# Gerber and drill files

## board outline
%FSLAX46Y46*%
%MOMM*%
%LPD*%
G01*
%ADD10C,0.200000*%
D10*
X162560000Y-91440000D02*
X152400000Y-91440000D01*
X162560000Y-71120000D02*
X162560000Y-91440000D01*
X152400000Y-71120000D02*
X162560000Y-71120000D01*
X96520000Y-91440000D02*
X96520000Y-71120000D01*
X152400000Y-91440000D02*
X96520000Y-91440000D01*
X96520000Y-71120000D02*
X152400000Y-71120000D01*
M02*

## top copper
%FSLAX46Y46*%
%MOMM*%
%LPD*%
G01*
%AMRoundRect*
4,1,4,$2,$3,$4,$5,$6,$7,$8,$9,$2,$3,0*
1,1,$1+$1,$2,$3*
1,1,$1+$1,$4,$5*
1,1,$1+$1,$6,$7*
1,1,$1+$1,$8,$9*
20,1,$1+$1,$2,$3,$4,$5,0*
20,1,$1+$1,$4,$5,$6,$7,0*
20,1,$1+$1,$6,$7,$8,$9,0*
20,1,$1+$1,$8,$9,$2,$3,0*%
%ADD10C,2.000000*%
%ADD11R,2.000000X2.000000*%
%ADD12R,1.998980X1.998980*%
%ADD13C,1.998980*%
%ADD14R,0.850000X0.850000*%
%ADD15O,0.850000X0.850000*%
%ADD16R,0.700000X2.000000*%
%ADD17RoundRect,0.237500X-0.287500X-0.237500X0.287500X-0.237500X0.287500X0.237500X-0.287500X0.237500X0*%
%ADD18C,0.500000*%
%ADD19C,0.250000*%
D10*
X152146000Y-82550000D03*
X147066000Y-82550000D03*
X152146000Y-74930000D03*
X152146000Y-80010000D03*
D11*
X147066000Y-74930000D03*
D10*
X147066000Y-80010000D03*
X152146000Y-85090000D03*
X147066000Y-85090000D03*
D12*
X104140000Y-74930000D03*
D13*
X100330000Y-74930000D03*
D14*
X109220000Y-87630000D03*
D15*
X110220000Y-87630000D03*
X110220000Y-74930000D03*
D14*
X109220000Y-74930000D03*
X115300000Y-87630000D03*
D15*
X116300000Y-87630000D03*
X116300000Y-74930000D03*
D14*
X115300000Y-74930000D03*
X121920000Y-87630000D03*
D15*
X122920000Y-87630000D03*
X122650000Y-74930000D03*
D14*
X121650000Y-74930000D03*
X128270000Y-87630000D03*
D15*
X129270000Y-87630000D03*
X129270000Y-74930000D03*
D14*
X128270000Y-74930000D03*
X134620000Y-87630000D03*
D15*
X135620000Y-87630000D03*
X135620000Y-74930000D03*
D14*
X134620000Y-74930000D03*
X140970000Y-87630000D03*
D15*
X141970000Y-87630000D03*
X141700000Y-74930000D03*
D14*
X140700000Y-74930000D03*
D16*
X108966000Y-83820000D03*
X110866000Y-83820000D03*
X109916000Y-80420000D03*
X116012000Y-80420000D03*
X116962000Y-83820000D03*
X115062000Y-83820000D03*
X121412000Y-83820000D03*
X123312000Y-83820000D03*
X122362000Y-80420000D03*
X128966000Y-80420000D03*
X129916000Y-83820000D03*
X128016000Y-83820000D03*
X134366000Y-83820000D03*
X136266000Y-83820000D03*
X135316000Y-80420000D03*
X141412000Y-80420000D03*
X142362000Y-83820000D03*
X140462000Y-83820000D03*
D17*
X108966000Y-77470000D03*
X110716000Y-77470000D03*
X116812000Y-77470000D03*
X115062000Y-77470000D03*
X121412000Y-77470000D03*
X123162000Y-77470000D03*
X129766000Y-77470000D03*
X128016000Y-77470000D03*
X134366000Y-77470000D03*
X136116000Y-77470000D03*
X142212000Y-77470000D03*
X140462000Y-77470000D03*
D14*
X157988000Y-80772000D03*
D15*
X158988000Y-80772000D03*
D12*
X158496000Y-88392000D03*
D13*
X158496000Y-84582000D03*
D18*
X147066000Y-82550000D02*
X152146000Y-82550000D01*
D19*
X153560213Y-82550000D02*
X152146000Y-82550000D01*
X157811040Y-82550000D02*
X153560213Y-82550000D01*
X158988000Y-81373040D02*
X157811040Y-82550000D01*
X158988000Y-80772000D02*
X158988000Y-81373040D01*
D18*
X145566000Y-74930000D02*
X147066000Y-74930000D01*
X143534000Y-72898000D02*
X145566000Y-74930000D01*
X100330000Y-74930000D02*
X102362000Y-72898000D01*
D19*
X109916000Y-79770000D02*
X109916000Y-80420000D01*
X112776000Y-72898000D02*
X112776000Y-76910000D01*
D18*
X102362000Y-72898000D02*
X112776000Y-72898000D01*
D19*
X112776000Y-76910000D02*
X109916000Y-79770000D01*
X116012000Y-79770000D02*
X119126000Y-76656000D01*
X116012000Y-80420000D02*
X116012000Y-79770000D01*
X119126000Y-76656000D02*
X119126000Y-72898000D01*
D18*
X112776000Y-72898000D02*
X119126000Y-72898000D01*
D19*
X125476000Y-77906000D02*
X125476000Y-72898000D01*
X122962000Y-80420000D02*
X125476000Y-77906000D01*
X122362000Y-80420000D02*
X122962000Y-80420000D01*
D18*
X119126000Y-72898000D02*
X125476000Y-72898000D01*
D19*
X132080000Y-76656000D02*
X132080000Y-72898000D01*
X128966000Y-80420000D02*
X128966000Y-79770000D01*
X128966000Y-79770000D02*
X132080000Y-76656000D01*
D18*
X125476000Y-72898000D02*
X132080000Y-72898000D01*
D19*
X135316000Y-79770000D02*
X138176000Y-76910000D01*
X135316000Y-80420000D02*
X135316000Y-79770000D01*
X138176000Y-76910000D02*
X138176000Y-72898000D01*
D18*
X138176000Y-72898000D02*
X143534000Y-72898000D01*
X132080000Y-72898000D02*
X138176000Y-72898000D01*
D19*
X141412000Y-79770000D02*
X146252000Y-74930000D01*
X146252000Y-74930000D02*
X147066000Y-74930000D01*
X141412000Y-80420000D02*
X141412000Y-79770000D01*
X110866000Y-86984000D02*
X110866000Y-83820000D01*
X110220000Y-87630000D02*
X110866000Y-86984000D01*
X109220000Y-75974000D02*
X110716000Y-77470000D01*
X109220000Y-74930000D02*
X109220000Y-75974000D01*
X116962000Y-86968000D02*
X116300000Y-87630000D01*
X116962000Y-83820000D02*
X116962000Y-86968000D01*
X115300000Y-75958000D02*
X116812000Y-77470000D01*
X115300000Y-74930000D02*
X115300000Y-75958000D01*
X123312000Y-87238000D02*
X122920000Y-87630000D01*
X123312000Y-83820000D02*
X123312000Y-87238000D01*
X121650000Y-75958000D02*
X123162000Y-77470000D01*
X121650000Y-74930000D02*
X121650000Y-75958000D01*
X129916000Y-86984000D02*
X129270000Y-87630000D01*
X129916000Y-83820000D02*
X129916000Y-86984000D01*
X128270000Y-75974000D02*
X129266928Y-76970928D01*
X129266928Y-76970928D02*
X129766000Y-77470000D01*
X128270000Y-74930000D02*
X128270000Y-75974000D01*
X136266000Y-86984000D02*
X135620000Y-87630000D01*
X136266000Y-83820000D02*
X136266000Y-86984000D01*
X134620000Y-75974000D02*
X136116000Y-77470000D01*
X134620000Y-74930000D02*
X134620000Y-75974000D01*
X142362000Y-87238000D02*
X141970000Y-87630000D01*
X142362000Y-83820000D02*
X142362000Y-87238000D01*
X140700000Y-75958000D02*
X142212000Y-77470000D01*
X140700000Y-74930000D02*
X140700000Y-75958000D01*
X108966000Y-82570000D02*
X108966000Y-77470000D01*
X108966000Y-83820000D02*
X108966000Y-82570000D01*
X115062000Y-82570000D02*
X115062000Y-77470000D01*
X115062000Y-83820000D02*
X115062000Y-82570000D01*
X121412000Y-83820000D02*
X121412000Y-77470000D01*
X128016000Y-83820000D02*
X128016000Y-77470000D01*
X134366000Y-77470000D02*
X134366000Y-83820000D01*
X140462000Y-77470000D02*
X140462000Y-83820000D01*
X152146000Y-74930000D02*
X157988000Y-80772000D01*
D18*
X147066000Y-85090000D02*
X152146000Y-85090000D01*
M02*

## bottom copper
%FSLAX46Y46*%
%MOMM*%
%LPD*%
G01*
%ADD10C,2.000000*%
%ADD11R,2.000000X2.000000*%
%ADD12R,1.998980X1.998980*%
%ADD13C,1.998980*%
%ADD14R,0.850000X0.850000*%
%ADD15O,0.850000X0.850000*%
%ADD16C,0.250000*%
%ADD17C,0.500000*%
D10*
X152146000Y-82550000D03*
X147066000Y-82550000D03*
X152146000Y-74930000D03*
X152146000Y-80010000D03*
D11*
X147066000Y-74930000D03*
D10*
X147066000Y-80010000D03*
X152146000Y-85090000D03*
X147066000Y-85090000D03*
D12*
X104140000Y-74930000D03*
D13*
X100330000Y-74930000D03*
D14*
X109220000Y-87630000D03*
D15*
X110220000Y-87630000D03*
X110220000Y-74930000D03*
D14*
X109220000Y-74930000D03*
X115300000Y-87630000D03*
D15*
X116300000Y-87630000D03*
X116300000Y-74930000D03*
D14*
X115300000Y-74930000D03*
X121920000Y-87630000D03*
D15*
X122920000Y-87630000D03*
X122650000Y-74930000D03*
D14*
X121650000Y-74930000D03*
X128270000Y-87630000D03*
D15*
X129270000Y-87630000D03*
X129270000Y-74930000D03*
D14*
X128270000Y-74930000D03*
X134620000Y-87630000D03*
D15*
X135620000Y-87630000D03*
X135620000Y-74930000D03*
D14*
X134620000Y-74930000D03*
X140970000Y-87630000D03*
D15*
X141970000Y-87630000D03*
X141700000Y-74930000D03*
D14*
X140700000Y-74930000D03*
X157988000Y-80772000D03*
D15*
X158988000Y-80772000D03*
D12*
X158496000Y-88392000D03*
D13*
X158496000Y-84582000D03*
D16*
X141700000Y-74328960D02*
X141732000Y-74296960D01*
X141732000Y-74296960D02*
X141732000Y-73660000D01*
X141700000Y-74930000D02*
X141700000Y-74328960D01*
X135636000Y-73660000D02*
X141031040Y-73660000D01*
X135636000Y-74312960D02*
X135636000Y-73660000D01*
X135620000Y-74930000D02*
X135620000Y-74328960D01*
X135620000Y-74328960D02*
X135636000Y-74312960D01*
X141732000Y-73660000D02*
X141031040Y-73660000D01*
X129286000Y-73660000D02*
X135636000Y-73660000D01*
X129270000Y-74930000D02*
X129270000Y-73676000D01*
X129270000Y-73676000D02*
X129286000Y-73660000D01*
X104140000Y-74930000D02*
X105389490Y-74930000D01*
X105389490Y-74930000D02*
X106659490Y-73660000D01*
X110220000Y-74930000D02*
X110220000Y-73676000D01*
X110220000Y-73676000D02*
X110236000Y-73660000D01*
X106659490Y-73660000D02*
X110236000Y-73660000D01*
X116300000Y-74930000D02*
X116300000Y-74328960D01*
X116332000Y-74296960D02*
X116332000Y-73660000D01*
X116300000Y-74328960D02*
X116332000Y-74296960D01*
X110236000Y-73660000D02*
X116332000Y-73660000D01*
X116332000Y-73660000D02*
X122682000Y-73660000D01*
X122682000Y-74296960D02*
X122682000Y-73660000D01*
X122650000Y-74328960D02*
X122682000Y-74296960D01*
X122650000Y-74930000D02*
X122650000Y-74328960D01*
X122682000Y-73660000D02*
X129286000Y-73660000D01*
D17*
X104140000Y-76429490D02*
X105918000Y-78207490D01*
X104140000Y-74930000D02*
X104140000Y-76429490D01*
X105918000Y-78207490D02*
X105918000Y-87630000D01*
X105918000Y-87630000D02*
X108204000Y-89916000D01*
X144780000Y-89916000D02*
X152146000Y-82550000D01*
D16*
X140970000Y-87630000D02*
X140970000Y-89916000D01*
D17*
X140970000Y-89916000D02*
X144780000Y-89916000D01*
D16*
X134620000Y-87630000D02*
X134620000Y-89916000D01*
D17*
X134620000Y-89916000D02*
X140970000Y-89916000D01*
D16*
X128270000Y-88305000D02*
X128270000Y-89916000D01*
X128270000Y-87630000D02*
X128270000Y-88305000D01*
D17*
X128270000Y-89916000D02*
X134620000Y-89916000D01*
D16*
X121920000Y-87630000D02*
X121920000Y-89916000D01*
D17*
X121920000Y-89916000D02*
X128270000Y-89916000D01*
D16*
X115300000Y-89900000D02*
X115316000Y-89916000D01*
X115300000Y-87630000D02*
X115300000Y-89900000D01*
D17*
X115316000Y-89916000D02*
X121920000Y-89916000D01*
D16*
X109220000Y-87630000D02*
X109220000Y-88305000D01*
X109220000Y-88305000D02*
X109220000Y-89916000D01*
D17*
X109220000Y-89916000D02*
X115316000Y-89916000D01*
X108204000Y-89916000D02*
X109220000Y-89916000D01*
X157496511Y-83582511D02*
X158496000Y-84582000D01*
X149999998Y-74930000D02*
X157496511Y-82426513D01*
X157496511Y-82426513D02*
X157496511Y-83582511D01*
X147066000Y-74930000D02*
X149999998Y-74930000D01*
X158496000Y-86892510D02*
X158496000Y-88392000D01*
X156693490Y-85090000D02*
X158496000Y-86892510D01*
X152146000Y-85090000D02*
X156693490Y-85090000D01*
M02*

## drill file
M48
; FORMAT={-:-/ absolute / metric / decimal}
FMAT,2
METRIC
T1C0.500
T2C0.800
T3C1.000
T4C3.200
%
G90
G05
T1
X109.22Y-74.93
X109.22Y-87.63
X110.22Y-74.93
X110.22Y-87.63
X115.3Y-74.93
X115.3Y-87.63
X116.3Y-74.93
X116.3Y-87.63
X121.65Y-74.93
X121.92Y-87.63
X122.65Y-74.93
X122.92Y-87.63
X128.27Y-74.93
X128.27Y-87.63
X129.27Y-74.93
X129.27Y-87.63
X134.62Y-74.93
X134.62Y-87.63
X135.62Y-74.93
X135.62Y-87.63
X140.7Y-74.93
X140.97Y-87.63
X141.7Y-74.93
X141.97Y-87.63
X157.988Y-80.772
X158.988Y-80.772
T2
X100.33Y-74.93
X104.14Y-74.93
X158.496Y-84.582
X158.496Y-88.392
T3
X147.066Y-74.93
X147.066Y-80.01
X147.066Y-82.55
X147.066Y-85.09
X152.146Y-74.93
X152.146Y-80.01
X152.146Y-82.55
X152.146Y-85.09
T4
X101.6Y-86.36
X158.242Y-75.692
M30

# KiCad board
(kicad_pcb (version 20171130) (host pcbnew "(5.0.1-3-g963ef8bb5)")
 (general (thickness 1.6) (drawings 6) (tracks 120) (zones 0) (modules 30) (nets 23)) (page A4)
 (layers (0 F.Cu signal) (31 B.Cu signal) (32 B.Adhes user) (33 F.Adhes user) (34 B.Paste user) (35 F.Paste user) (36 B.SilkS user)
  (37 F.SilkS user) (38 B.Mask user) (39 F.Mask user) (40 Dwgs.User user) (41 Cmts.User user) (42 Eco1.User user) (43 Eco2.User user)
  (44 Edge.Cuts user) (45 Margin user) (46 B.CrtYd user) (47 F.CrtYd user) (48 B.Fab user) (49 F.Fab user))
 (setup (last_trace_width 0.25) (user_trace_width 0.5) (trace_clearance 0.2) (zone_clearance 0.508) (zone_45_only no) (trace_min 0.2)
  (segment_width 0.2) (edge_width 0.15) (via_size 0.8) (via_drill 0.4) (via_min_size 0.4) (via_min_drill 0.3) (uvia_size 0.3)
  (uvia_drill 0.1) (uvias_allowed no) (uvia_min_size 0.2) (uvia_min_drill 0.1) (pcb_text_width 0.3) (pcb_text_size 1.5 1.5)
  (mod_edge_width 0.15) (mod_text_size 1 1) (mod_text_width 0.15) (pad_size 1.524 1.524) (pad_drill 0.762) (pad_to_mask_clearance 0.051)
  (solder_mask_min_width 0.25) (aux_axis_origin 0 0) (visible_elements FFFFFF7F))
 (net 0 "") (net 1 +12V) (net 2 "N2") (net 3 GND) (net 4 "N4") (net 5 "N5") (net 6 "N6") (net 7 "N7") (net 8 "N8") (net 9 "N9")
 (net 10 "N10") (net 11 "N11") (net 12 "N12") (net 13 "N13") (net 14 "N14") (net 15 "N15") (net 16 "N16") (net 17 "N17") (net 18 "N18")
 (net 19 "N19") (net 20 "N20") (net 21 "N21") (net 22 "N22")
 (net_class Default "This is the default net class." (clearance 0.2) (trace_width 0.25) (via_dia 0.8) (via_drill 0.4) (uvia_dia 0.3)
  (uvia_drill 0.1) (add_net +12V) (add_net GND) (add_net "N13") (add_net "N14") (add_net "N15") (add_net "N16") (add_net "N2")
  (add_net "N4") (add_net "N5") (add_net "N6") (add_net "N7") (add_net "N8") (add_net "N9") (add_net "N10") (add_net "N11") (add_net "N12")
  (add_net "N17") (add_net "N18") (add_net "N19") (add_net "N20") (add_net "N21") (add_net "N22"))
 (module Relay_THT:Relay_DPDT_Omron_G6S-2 (layer F.Cu) (at 147.066 74.93)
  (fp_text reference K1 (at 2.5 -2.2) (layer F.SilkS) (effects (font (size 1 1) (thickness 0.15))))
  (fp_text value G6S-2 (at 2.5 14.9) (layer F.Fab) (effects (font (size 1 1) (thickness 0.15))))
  (pad 7 thru_hole circle (at 5.08 7.62 270) (size 2 2) (drill 1) (layers *.Cu *.Mask) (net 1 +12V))
  (pad 4 thru_hole circle (at 0 7.62 270) (size 2 2) (drill 1) (layers *.Cu *.Mask) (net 1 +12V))
  (pad 10 thru_hole circle (at 5.08 0) (size 2 2) (drill 1) (layers *.Cu *.Mask) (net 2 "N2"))
  (pad 8 thru_hole circle (at 5.08 5.08) (size 2 2) (drill 1) (layers *.Cu *.Mask))
  (pad 1 thru_hole rect (at 0 0) (size 2 2) (drill 1) (layers *.Cu *.Mask) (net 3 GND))
  (pad 3 thru_hole circle (at 0 5.08) (size 2 2) (drill 1) (layers *.Cu *.Mask))
  (pad 6 thru_hole circle (at 5.08 10.16) (size 2 2) (drill 1) (layers *.Cu *.Mask) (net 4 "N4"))
  (pad 5 thru_hole circle (at 0 10.16) (size 2 2) (drill 1) (layers *.Cu *.Mask) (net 4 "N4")))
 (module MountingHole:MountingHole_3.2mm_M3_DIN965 (layer F.Cu) (at 101.6 86.36)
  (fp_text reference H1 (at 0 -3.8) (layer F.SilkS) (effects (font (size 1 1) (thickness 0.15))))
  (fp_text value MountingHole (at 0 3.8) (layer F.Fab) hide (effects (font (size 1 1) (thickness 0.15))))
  (pad 1 np_thru_hole circle (at 0 0) (size 3.2 3.2) (drill 3.2) (layers *.Cu *.Mask)))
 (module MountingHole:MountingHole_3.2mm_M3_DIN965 (layer F.Cu) (at 158.242 75.692)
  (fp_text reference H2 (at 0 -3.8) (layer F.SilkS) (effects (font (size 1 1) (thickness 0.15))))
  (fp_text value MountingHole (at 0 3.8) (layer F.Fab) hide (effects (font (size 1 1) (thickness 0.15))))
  (pad 1 np_thru_hole circle (at 0 0) (size 3.2 3.2) (drill 3.2) (layers *.Cu *.Mask)))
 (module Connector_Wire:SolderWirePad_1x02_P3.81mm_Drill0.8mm (layer F.Cu) (at 104.14 74.93 180)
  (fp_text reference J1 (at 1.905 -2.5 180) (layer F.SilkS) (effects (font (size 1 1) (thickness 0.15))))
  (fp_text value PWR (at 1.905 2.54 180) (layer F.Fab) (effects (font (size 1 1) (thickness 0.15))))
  (pad 1 thru_hole rect (at 0 0 180) (size 1.99898 1.99898) (drill 0.8001) (layers *.Cu *.Mask) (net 1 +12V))
  (pad 2 thru_hole circle (at 3.81 0 180) (size 1.99898 1.99898) (drill 0.8001) (layers *.Cu *.Mask) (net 3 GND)))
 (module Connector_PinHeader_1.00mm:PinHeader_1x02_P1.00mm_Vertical (layer F.Cu) (at 109.22 87.63 90)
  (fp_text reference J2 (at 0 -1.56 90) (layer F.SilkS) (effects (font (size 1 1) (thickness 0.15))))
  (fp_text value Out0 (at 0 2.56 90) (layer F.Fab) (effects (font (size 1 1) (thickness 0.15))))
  (pad 1 thru_hole rect (at 0 0 90) (size 0.85 0.85) (drill 0.5) (layers *.Cu *.Mask) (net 1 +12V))
  (pad 2 thru_hole oval (at 0 1 90) (size 0.85 0.85) (drill 0.5) (layers *.Cu *.Mask) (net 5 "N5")))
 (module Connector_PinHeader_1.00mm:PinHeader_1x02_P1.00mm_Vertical (layer F.Cu) (at 109.22 74.93 90)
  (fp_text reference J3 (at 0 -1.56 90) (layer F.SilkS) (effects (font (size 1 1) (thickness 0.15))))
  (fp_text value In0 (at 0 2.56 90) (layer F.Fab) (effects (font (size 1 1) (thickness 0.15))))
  (pad 2 thru_hole oval (at 0 1 90) (size 0.85 0.85) (drill 0.5) (layers *.Cu *.Mask) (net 1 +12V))
  (pad 1 thru_hole rect (at 0 0 90) (size 0.85 0.85) (drill 0.5) (layers *.Cu *.Mask) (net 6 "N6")))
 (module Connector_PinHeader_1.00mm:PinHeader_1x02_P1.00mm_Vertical (layer F.Cu) (at 115.3 87.63 90)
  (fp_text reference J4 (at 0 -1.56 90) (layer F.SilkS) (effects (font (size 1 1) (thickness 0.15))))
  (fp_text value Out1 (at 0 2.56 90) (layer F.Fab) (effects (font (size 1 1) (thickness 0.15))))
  (pad 1 thru_hole rect (at 0 0 90) (size 0.85 0.85) (drill 0.5) (layers *.Cu *.Mask) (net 1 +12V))
  (pad 2 thru_hole oval (at 0 1 90) (size 0.85 0.85) (drill 0.5) (layers *.Cu *.Mask) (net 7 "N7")))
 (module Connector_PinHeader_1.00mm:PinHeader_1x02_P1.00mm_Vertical (layer F.Cu) (at 115.3 74.93 90)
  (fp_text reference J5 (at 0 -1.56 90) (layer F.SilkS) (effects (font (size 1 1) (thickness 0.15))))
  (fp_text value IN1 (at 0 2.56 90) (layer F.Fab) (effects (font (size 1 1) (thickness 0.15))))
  (pad 2 thru_hole oval (at 0 1 90) (size 0.85 0.85) (drill 0.5) (layers *.Cu *.Mask) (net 1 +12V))
  (pad 1 thru_hole rect (at 0 0 90) (size 0.85 0.85) (drill 0.5) (layers *.Cu *.Mask) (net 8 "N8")))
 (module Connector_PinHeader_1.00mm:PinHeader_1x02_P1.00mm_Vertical (layer F.Cu) (at 121.92 87.63 90)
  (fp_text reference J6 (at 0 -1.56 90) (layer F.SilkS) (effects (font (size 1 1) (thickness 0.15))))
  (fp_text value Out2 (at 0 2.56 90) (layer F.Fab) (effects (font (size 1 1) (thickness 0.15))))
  (pad 1 thru_hole rect (at 0 0 90) (size 0.85 0.85) (drill 0.5) (layers *.Cu *.Mask) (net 1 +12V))
  (pad 2 thru_hole oval (at 0 1 90) (size 0.85 0.85) (drill 0.5) (layers *.Cu *.Mask) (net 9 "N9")))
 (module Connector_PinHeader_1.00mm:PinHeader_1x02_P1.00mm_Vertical (layer F.Cu) (at 121.65 74.93 90)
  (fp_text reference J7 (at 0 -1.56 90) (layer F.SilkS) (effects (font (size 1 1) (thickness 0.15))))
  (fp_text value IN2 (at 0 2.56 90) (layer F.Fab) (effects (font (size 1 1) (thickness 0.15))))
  (pad 2 thru_hole oval (at 0 1 90) (size 0.85 0.85) (drill 0.5) (layers *.Cu *.Mask) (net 1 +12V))
  (pad 1 thru_hole rect (at 0 0 90) (size 0.85 0.85) (drill 0.5) (layers *.Cu *.Mask) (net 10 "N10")))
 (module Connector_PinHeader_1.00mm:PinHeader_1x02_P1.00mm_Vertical (layer F.Cu) (at 128.27 87.63 90)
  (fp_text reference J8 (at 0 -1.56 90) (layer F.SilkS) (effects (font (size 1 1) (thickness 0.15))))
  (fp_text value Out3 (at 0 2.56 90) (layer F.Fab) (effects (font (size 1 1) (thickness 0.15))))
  (pad 1 thru_hole rect (at 0 0 90) (size 0.85 0.85) (drill 0.5) (layers *.Cu *.Mask) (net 1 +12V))
  (pad 2 thru_hole oval (at 0 1 90) (size 0.85 0.85) (drill 0.5) (layers *.Cu *.Mask) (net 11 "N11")))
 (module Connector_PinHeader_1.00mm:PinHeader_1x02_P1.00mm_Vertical (layer F.Cu) (at 128.27 74.93 90)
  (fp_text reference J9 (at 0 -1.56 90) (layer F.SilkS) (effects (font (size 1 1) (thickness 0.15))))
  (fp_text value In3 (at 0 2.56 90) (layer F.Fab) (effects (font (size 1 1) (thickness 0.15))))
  (pad 2 thru_hole oval (at 0 1 90) (size 0.85 0.85) (drill 0.5) (layers *.Cu *.Mask) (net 1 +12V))
  (pad 1 thru_hole rect (at 0 0 90) (size 0.85 0.85) (drill 0.5) (layers *.Cu *.Mask) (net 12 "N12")))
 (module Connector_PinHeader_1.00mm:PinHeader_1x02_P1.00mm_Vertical (layer F.Cu) (at 134.62 87.63 90)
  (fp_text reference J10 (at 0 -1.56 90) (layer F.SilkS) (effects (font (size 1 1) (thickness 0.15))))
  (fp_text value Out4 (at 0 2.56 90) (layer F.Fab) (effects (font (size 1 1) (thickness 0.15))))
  (pad 1 thru_hole rect (at 0 0 90) (size 0.85 0.85) (drill 0.5) (layers *.Cu *.Mask) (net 1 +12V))
  (pad 2 thru_hole oval (at 0 1 90) (size 0.85 0.85) (drill 0.5) (layers *.Cu *.Mask) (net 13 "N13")))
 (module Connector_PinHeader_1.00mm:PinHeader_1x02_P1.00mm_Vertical (layer F.Cu) (at 134.62 74.93 90)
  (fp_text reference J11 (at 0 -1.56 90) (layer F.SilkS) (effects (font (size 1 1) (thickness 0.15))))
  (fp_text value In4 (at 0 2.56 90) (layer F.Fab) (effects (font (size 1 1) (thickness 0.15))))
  (pad 2 thru_hole oval (at 0 1 90) (size 0.85 0.85) (drill 0.5) (layers *.Cu *.Mask) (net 1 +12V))
  (pad 1 thru_hole rect (at 0 0 90) (size 0.85 0.85) (drill 0.5) (layers *.Cu *.Mask) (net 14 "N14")))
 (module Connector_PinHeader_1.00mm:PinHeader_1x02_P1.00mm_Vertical (layer F.Cu) (at 140.97 87.63 90)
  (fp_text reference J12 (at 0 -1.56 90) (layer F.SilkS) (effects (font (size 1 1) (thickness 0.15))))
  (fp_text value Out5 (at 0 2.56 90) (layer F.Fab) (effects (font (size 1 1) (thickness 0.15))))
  (pad 1 thru_hole rect (at 0 0 90) (size 0.85 0.85) (drill 0.5) (layers *.Cu *.Mask) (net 1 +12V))
  (pad 2 thru_hole oval (at 0 1 90) (size 0.85 0.85) (drill 0.5) (layers *.Cu *.Mask) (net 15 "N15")))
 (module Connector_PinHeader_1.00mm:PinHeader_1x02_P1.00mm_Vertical (layer F.Cu) (at 140.7 74.93 90)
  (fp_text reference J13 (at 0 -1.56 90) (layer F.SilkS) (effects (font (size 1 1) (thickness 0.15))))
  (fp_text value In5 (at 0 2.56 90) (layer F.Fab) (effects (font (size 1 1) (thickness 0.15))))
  (pad 2 thru_hole oval (at 0 1 90) (size 0.85 0.85) (drill 0.5) (layers *.Cu *.Mask) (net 1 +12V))
  (pad 1 thru_hole rect (at 0 0 90) (size 0.85 0.85) (drill 0.5) (layers *.Cu *.Mask) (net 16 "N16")))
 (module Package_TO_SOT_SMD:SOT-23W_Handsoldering (layer F.Cu) (at 109.916 82.12 90)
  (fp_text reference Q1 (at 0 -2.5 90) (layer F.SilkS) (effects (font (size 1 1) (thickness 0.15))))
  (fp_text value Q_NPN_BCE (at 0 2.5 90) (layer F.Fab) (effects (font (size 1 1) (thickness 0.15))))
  (pad 1 smd rect (at -1.7 -0.95 90) (size 2 0.7) (layers F.Cu F.Paste F.Mask) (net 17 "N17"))
  (pad 2 smd rect (at -1.7 0.95 90) (size 2 0.7) (layers F.Cu F.Paste F.Mask) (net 5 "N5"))
  (pad 3 smd rect (at 1.7 0 90) (size 2 0.7) (layers F.Cu F.Paste F.Mask) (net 3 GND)))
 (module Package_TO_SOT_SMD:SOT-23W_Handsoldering (layer F.Cu) (at 116.012 82.12 90)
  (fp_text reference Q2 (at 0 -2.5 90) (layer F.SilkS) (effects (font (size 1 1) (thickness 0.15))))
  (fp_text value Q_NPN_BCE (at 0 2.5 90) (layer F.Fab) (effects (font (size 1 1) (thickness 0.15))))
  (pad 3 smd rect (at 1.7 0 90) (size 2 0.7) (layers F.Cu F.Paste F.Mask) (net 3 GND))
  (pad 2 smd rect (at -1.7 0.95 90) (size 2 0.7) (layers F.Cu F.Paste F.Mask) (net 7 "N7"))
  (pad 1 smd rect (at -1.7 -0.95 90) (size 2 0.7) (layers F.Cu F.Paste F.Mask) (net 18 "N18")))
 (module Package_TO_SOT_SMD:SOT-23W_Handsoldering (layer F.Cu) (at 122.362 82.12 90)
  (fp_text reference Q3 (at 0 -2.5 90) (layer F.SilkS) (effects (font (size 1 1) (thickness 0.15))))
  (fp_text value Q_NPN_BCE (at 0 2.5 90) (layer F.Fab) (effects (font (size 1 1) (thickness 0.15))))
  (pad 1 smd rect (at -1.7 -0.95 90) (size 2 0.7) (layers F.Cu F.Paste F.Mask) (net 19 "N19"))
  (pad 2 smd rect (at -1.7 0.95 90) (size 2 0.7) (layers F.Cu F.Paste F.Mask) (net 9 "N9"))
  (pad 3 smd rect (at 1.7 0 90) (size 2 0.7) (layers F.Cu F.Paste F.Mask) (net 3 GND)))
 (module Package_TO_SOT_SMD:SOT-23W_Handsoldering (layer F.Cu) (at 128.966 82.12 90)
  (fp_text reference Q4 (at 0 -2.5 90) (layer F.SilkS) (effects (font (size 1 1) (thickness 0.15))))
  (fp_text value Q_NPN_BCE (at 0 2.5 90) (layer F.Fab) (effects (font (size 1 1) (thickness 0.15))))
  (pad 3 smd rect (at 1.7 0 90) (size 2 0.7) (layers F.Cu F.Paste F.Mask) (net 3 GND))
  (pad 2 smd rect (at -1.7 0.95 90) (size 2 0.7) (layers F.Cu F.Paste F.Mask) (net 11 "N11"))
  (pad 1 smd rect (at -1.7 -0.95 90) (size 2 0.7) (layers F.Cu F.Paste F.Mask) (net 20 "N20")))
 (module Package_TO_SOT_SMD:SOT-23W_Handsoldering (layer F.Cu) (at 135.316 82.12 90)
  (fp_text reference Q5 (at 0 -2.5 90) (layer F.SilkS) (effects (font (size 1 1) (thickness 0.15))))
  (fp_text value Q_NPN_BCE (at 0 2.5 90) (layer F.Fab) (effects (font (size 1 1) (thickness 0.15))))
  (pad 1 smd rect (at -1.7 -0.95 90) (size 2 0.7) (layers F.Cu F.Paste F.Mask) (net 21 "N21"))
  (pad 2 smd rect (at -1.7 0.95 90) (size 2 0.7) (layers F.Cu F.Paste F.Mask) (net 13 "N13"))
  (pad 3 smd rect (at 1.7 0 90) (size 2 0.7) (layers F.Cu F.Paste F.Mask) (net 3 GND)))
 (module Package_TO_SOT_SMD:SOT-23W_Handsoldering (layer F.Cu) (at 141.412 82.12 90)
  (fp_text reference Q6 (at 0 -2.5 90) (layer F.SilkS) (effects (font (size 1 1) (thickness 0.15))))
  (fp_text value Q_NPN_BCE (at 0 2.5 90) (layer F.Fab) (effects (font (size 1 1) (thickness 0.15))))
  (pad 3 smd rect (at 1.7 0 90) (size 2 0.7) (layers F.Cu F.Paste F.Mask) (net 3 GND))
  (pad 2 smd rect (at -1.7 0.95 90) (size 2 0.7) (layers F.Cu F.Paste F.Mask) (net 15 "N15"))
  (pad 1 smd rect (at -1.7 -0.95 90) (size 2 0.7) (layers F.Cu F.Paste F.Mask) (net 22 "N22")))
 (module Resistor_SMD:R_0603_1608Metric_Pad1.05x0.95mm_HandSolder (layer F.Cu) (at 109.841 77.47)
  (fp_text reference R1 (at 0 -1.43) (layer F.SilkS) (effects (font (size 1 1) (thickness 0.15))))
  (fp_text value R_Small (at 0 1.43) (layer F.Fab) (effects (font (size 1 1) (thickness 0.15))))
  (pad 1 smd roundrect (at -0.875 0) (size 1.05 0.95) (layers F.Cu F.Paste F.Mask) (roundrect_rratio 0.25) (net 17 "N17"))
  (pad 2 smd roundrect (at 0.875 0) (size 1.05 0.95) (layers F.Cu F.Paste F.Mask) (roundrect_rratio 0.25) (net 6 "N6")))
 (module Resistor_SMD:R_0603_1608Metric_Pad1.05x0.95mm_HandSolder (layer F.Cu) (at 115.937 77.47)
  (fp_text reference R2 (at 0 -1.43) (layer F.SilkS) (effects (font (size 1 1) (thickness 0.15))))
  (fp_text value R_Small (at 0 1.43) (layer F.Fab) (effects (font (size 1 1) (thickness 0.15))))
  (pad 2 smd roundrect (at 0.875 0) (size 1.05 0.95) (layers F.Cu F.Paste F.Mask) (roundrect_rratio 0.25) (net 8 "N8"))
  (pad 1 smd roundrect (at -0.875 0) (size 1.05 0.95) (layers F.Cu F.Paste F.Mask) (roundrect_rratio 0.25) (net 18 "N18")))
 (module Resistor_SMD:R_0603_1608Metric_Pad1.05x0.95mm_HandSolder (layer F.Cu) (at 122.287 77.47)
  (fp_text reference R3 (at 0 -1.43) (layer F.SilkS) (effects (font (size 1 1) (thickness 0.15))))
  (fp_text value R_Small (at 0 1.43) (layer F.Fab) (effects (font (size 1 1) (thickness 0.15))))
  (pad 1 smd roundrect (at -0.875 0) (size 1.05 0.95) (layers F.Cu F.Paste F.Mask) (roundrect_rratio 0.25) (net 19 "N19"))
  (pad 2 smd roundrect (at 0.875 0) (size 1.05 0.95) (layers F.Cu F.Paste F.Mask) (roundrect_rratio 0.25) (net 10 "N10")))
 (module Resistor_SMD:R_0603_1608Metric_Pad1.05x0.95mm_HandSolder (layer F.Cu) (at 128.891 77.47)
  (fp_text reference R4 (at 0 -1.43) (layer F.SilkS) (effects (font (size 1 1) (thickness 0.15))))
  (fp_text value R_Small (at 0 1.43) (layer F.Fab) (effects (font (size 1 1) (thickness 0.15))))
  (pad 2 smd roundrect (at 0.875 0) (size 1.05 0.95) (layers F.Cu F.Paste F.Mask) (roundrect_rratio 0.25) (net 12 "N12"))
  (pad 1 smd roundrect (at -0.875 0) (size 1.05 0.95) (layers F.Cu F.Paste F.Mask) (roundrect_rratio 0.25) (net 20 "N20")))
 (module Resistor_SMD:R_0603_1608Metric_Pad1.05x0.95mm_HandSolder (layer F.Cu) (at 135.241 77.47)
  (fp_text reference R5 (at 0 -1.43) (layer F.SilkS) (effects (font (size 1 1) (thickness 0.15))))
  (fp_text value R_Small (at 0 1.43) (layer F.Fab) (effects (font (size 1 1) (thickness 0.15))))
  (pad 1 smd roundrect (at -0.875 0) (size 1.05 0.95) (layers F.Cu F.Paste F.Mask) (roundrect_rratio 0.25) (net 21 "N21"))
  (pad 2 smd roundrect (at 0.875 0) (size 1.05 0.95) (layers F.Cu F.Paste F.Mask) (roundrect_rratio 0.25) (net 14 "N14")))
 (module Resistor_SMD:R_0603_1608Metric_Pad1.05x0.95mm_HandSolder (layer F.Cu) (at 141.337 77.47)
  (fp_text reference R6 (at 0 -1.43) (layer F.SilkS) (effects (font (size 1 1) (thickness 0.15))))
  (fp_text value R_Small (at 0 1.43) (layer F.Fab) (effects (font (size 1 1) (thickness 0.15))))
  (pad 2 smd roundrect (at 0.875 0) (size 1.05 0.95) (layers F.Cu F.Paste F.Mask) (roundrect_rratio 0.25) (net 16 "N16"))
  (pad 1 smd roundrect (at -0.875 0) (size 1.05 0.95) (layers F.Cu F.Paste F.Mask) (roundrect_rratio 0.25) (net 22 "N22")))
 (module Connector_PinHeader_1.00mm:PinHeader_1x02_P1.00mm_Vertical (layer F.Cu) (at 157.988 80.772 90)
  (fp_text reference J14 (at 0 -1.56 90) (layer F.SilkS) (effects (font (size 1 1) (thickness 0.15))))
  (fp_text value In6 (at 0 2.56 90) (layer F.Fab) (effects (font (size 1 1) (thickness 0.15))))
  (pad 1 thru_hole rect (at 0 0 90) (size 0.85 0.85) (drill 0.5) (layers *.Cu *.Mask) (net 2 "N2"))
  (pad 2 thru_hole oval (at 0 1 90) (size 0.85 0.85) (drill 0.5) (layers *.Cu *.Mask) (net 1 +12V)))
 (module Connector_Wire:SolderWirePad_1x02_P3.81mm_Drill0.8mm (layer F.Cu) (at 158.496 88.392 90)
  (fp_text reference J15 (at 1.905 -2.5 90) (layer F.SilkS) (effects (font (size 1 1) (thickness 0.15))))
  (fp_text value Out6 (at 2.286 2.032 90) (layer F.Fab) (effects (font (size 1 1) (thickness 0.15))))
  (pad 1 thru_hole rect (at 0 0 90) (size 1.99898 1.99898) (drill 0.8001) (layers *.Cu *.Mask) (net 4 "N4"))
  (pad 2 thru_hole circle (at 3.81 0 90) (size 1.99898 1.99898) (drill 0.8001) (layers *.Cu *.Mask) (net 3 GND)))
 (gr_line (start 162.56 91.44) (end 152.4 91.44) (layer Edge.Cuts) (width 0.2))
 (gr_line (start 162.56 71.12) (end 162.56 91.44) (layer Edge.Cuts) (width 0.2))
 (gr_line (start 152.4 71.12) (end 162.56 71.12) (layer Edge.Cuts) (width 0.2))
 (gr_line (start 96.52 91.44) (end 96.52 71.12) (layer Edge.Cuts) (width 0.2))
 (gr_line (start 152.4 91.44) (end 96.52 91.44) (layer Edge.Cuts) (width 0.2))
 (gr_line (start 96.52 71.12) (end 152.4 71.12) (layer Edge.Cuts) (width 0.2))
 (segment (start 147.066 82.55) (end 152.146 82.55) (width 0.5) (layer F.Cu) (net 1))
 (segment (start 141.7 74.32896) (end 141.732 74.29696) (width 0.25) (layer B.Cu) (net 1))
 (segment (start 141.732 74.29696) (end 141.732 73.66) (width 0.25) (layer B.Cu) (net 1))
 (segment (start 141.7 74.93) (end 141.7 74.32896) (width 0.25) (layer B.Cu) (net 1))
 (segment (start 135.636 73.66) (end 141.03104 73.66) (width 0.25) (layer B.Cu) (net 1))
 (segment (start 135.636 74.31296) (end 135.636 73.66) (width 0.25) (layer B.Cu) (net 1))
 (segment (start 135.62 74.93) (end 135.62 74.32896) (width 0.25) (layer B.Cu) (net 1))
 (segment (start 135.62 74.32896) (end 135.636 74.31296) (width 0.25) (layer B.Cu) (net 1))
 (segment (start 141.732 73.66) (end 141.03104 73.66) (width 0.25) (layer B.Cu) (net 1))
 (segment (start 129.286 73.66) (end 135.636 73.66) (width 0.25) (layer B.Cu) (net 1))
 (segment (start 129.27 74.93) (end 129.27 73.676) (width 0.25) (layer B.Cu) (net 1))
 (segment (start 129.27 73.676) (end 129.286 73.66) (width 0.25) (layer B.Cu) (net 1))
 (segment (start 104.14 74.93) (end 105.38949 74.93) (width 0.25) (layer B.Cu) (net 1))
 (segment (start 105.38949 74.93) (end 106.65949 73.66) (width 0.25) (layer B.Cu) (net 1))
 (segment (start 110.22 74.93) (end 110.22 73.676) (width 0.25) (layer B.Cu) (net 1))
 (segment (start 110.22 73.676) (end 110.236 73.66) (width 0.25) (layer B.Cu) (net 1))
 (segment (start 106.65949 73.66) (end 110.236 73.66) (width 0.25) (layer B.Cu) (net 1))
 (segment (start 116.3 74.93) (end 116.3 74.32896) (width 0.25) (layer B.Cu) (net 1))
 (segment (start 116.332 74.29696) (end 116.332 73.66) (width 0.25) (layer B.Cu) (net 1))
 (segment (start 116.3 74.32896) (end 116.332 74.29696) (width 0.25) (layer B.Cu) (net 1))
 (segment (start 110.236 73.66) (end 116.332 73.66) (width 0.25) (layer B.Cu) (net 1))
 (segment (start 116.332 73.66) (end 122.682 73.66) (width 0.25) (layer B.Cu) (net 1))
 (segment (start 122.682 74.29696) (end 122.682 73.66) (width 0.25) (layer B.Cu) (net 1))
 (segment (start 122.65 74.32896) (end 122.682 74.29696) (width 0.25) (layer B.Cu) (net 1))
 (segment (start 122.65 74.93) (end 122.65 74.32896) (width 0.25) (layer B.Cu) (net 1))
 (segment (start 122.682 73.66) (end 129.286 73.66) (width 0.25) (layer B.Cu) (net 1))
 (segment (start 104.14 76.42949) (end 105.918 78.20749) (width 0.5) (layer B.Cu) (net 1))
 (segment (start 104.14 74.93) (end 104.14 76.42949) (width 0.5) (layer B.Cu) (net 1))
 (segment (start 105.918 78.20749) (end 105.918 87.63) (width 0.5) (layer B.Cu) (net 1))
 (segment (start 105.918 87.63) (end 108.204 89.916) (width 0.5) (layer B.Cu) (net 1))
 (segment (start 144.78 89.916) (end 152.146 82.55) (width 0.5) (layer B.Cu) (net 1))
 (segment (start 140.97 87.63) (end 140.97 89.916) (width 0.25) (layer B.Cu) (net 1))
 (segment (start 140.97 89.916) (end 144.78 89.916) (width 0.5) (layer B.Cu) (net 1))
 (segment (start 134.62 87.63) (end 134.62 89.916) (width 0.25) (layer B.Cu) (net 1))
 (segment (start 134.62 89.916) (end 140.97 89.916) (width 0.5) (layer B.Cu) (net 1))
 (segment (start 128.27 88.305) (end 128.27 89.916) (width 0.25) (layer B.Cu) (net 1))
 (segment (start 128.27 87.63) (end 128.27 88.305) (width 0.25) (layer B.Cu) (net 1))
 (segment (start 128.27 89.916) (end 134.62 89.916) (width 0.5) (layer B.Cu) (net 1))
 (segment (start 121.92 87.63) (end 121.92 89.916) (width 0.25) (layer B.Cu) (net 1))
 (segment (start 121.92 89.916) (end 128.27 89.916) (width 0.5) (layer B.Cu) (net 1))
 (segment (start 115.3 89.9) (end 115.316 89.916) (width 0.25) (layer B.Cu) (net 1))
 (segment (start 115.3 87.63) (end 115.3 89.9) (width 0.25) (layer B.Cu) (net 1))
 (segment (start 115.316 89.916) (end 121.92 89.916) (width 0.5) (layer B.Cu) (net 1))
 (segment (start 109.22 87.63) (end 109.22 88.305) (width 0.25) (layer B.Cu) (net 1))
 (segment (start 109.22 88.305) (end 109.22 89.916) (width 0.25) (layer B.Cu) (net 1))
 (segment (start 109.22 89.916) (end 115.316 89.916) (width 0.5) (layer B.Cu) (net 1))
 (segment (start 108.204 89.916) (end 109.22 89.916) (width 0.5) (layer B.Cu) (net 1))
 (segment (start 153.560213 82.55) (end 152.146 82.55) (width 0.25) (layer F.Cu) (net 1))
 (segment (start 157.81104 82.55) (end 153.560213 82.55) (width 0.25) (layer F.Cu) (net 1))
 (segment (start 158.988 81.37304) (end 157.81104 82.55) (width 0.25) (layer F.Cu) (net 1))
 (segment (start 158.988 80.772) (end 158.988 81.37304) (width 0.25) (layer F.Cu) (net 1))
 (segment (start 145.566 74.93) (end 147.066 74.93) (width 0.5) (layer F.Cu) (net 3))
 (segment (start 143.534 72.898) (end 145.566 74.93) (width 0.5) (layer F.Cu) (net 3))
 (segment (start 100.33 74.93) (end 102.362 72.898) (width 0.5) (layer F.Cu) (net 3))
 (segment (start 109.916 79.77) (end 109.916 80.42) (width 0.25) (layer F.Cu) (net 3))
 (segment (start 112.776 72.898) (end 112.776 76.91) (width 0.25) (layer F.Cu) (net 3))
 (segment (start 102.362 72.898) (end 112.776 72.898) (width 0.5) (layer F.Cu) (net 3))
 (segment (start 112.776 76.91) (end 109.916 79.77) (width 0.25) (layer F.Cu) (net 3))
 (segment (start 116.012 79.77) (end 119.126 76.656) (width 0.25) (layer F.Cu) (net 3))
 (segment (start 116.012 80.42) (end 116.012 79.77) (width 0.25) (layer F.Cu) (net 3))
 (segment (start 119.126 76.656) (end 119.126 72.898) (width 0.25) (layer F.Cu) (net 3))
 (segment (start 112.776 72.898) (end 119.126 72.898) (width 0.5) (layer F.Cu) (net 3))
 (segment (start 125.476 77.906) (end 125.476 72.898) (width 0.25) (layer F.Cu) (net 3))
 (segment (start 122.962 80.42) (end 125.476 77.906) (width 0.25) (layer F.Cu) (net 3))
 (segment (start 122.362 80.42) (end 122.962 80.42) (width 0.25) (layer F.Cu) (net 3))
 (segment (start 119.126 72.898) (end 125.476 72.898) (width 0.5) (layer F.Cu) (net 3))
 (segment (start 132.08 76.656) (end 132.08 72.898) (width 0.25) (layer F.Cu) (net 3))
 (segment (start 128.966 80.42) (end 128.966 79.77) (width 0.25) (layer F.Cu) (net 3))
 (segment (start 128.966 79.77) (end 132.08 76.656) (width 0.25) (layer F.Cu) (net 3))
 (segment (start 125.476 72.898) (end 132.08 72.898) (width 0.5) (layer F.Cu) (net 3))
 (segment (start 135.316 79.77) (end 138.176 76.91) (width 0.25) (layer F.Cu) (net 3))
 (segment (start 135.316 80.42) (end 135.316 79.77) (width 0.25) (layer F.Cu) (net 3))
 (segment (start 138.176 76.91) (end 138.176 72.898) (width 0.25) (layer F.Cu) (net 3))
 (segment (start 138.176 72.898) (end 143.534 72.898) (width 0.5) (layer F.Cu) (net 3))
 (segment (start 132.08 72.898) (end 138.176 72.898) (width 0.5) (layer F.Cu) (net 3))
 (segment (start 141.412 79.77) (end 146.252 74.93) (width 0.25) (layer F.Cu) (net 3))
 (segment (start 146.252 74.93) (end 147.066 74.93) (width 0.25) (layer F.Cu) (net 3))
 (segment (start 141.412 80.42) (end 141.412 79.77) (width 0.25) (layer F.Cu) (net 3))
 (segment (start 157.496511 83.582511) (end 158.496 84.582) (width 0.5) (layer B.Cu) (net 3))
 (segment (start 149.999998 74.93) (end 157.496511 82.426513) (width 0.5) (layer B.Cu) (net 3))
 (segment (start 157.496511 82.426513) (end 157.496511 83.582511) (width 0.5) (layer B.Cu) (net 3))
 (segment (start 147.066 74.93) (end 149.999998 74.93) (width 0.5) (layer B.Cu) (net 3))
 (segment (start 110.866 86.984) (end 110.866 83.82) (width 0.25) (layer F.Cu) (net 5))
 (segment (start 110.22 87.63) (end 110.866 86.984) (width 0.25) (layer F.Cu) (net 5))
 (segment (start 109.22 75.974) (end 110.716 77.47) (width 0.25) (layer F.Cu) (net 6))
 (segment (start 109.22 74.93) (end 109.22 75.974) (width 0.25) (layer F.Cu) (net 6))
 (segment (start 116.962 86.968) (end 116.3 87.63) (width 0.25) (layer F.Cu) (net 7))
 (segment (start 116.962 83.82) (end 116.962 86.968) (width 0.25) (layer F.Cu) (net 7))
 (segment (start 115.3 75.958) (end 116.812 77.47) (width 0.25) (layer F.Cu) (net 8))
 (segment (start 115.3 74.93) (end 115.3 75.958) (width 0.25) (layer F.Cu) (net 8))
 (segment (start 123.312 87.238) (end 122.92 87.63) (width 0.25) (layer F.Cu) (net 9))
 (segment (start 123.312 83.82) (end 123.312 87.238) (width 0.25) (layer F.Cu) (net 9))
 (segment (start 121.65 75.958) (end 123.162 77.47) (width 0.25) (layer F.Cu) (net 10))
 (segment (start 121.65 74.93) (end 121.65 75.958) (width 0.25) (layer F.Cu) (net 10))
 (segment (start 129.916 86.984) (end 129.27 87.63) (width 0.25) (layer F.Cu) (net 11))
 (segment (start 129.916 83.82) (end 129.916 86.984) (width 0.25) (layer F.Cu) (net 11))
 (segment (start 128.27 75.974) (end 129.266928 76.970928) (width 0.25) (layer F.Cu) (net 12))
 (segment (start 129.266928 76.970928) (end 129.766 77.47) (width 0.25) (layer F.Cu) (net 12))
 (segment (start 128.27 74.93) (end 128.27 75.974) (width 0.25) (layer F.Cu) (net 12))
 (segment (start 136.266 86.984) (end 135.62 87.63) (width 0.25) (layer F.Cu) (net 13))
 (segment (start 136.266 83.82) (end 136.266 86.984) (width 0.25) (layer F.Cu) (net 13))
 (segment (start 134.62 75.974) (end 136.116 77.47) (width 0.25) (layer F.Cu) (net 14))
 (segment (start 134.62 74.93) (end 134.62 75.974) (width 0.25) (layer F.Cu) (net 14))
 (segment (start 142.362 87.238) (end 141.97 87.63) (width 0.25) (layer F.Cu) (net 15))
 (segment (start 142.362 83.82) (end 142.362 87.238) (width 0.25) (layer F.Cu) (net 15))
 (segment (start 140.7 75.958) (end 142.212 77.47) (width 0.25) (layer F.Cu) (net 16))
 (segment (start 140.7 74.93) (end 140.7 75.958) (width 0.25) (layer F.Cu) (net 16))
 (segment (start 108.966 82.57) (end 108.966 77.47) (width 0.25) (layer F.Cu) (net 17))
 (segment (start 108.966 83.82) (end 108.966 82.57) (width 0.25) (layer F.Cu) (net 17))
 (segment (start 115.062 82.57) (end 115.062 77.47) (width 0.25) (layer F.Cu) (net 18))
 (segment (start 115.062 83.82) (end 115.062 82.57) (width 0.25) (layer F.Cu) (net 18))
 (segment (start 121.412 83.82) (end 121.412 77.47) (width 0.25) (layer F.Cu) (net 19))
 (segment (start 128.016 83.82) (end 128.016 77.47) (width 0.25) (layer F.Cu) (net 20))
 (segment (start 134.366 77.47) (end 134.366 83.82) (width 0.25) (layer F.Cu) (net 21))
 (segment (start 140.462 77.47) (end 140.462 83.82) (width 0.25) (layer F.Cu) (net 22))
 (segment (start 152.146 74.93) (end 157.988 80.772) (width 0.25) (layer F.Cu) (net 2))
 (segment (start 147.066 85.09) (end 152.146 85.09) (width 0.5) (layer F.Cu) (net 4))
 (segment (start 158.496 86.89251) (end 158.496 88.392) (width 0.5) (layer B.Cu) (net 4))
 (segment (start 156.69349 85.09) (end 158.496 86.89251) (width 0.5) (layer B.Cu) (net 4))
 (segment (start 152.146 85.09) (end 156.69349 85.09) (width 0.5) (layer B.Cu) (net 4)))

